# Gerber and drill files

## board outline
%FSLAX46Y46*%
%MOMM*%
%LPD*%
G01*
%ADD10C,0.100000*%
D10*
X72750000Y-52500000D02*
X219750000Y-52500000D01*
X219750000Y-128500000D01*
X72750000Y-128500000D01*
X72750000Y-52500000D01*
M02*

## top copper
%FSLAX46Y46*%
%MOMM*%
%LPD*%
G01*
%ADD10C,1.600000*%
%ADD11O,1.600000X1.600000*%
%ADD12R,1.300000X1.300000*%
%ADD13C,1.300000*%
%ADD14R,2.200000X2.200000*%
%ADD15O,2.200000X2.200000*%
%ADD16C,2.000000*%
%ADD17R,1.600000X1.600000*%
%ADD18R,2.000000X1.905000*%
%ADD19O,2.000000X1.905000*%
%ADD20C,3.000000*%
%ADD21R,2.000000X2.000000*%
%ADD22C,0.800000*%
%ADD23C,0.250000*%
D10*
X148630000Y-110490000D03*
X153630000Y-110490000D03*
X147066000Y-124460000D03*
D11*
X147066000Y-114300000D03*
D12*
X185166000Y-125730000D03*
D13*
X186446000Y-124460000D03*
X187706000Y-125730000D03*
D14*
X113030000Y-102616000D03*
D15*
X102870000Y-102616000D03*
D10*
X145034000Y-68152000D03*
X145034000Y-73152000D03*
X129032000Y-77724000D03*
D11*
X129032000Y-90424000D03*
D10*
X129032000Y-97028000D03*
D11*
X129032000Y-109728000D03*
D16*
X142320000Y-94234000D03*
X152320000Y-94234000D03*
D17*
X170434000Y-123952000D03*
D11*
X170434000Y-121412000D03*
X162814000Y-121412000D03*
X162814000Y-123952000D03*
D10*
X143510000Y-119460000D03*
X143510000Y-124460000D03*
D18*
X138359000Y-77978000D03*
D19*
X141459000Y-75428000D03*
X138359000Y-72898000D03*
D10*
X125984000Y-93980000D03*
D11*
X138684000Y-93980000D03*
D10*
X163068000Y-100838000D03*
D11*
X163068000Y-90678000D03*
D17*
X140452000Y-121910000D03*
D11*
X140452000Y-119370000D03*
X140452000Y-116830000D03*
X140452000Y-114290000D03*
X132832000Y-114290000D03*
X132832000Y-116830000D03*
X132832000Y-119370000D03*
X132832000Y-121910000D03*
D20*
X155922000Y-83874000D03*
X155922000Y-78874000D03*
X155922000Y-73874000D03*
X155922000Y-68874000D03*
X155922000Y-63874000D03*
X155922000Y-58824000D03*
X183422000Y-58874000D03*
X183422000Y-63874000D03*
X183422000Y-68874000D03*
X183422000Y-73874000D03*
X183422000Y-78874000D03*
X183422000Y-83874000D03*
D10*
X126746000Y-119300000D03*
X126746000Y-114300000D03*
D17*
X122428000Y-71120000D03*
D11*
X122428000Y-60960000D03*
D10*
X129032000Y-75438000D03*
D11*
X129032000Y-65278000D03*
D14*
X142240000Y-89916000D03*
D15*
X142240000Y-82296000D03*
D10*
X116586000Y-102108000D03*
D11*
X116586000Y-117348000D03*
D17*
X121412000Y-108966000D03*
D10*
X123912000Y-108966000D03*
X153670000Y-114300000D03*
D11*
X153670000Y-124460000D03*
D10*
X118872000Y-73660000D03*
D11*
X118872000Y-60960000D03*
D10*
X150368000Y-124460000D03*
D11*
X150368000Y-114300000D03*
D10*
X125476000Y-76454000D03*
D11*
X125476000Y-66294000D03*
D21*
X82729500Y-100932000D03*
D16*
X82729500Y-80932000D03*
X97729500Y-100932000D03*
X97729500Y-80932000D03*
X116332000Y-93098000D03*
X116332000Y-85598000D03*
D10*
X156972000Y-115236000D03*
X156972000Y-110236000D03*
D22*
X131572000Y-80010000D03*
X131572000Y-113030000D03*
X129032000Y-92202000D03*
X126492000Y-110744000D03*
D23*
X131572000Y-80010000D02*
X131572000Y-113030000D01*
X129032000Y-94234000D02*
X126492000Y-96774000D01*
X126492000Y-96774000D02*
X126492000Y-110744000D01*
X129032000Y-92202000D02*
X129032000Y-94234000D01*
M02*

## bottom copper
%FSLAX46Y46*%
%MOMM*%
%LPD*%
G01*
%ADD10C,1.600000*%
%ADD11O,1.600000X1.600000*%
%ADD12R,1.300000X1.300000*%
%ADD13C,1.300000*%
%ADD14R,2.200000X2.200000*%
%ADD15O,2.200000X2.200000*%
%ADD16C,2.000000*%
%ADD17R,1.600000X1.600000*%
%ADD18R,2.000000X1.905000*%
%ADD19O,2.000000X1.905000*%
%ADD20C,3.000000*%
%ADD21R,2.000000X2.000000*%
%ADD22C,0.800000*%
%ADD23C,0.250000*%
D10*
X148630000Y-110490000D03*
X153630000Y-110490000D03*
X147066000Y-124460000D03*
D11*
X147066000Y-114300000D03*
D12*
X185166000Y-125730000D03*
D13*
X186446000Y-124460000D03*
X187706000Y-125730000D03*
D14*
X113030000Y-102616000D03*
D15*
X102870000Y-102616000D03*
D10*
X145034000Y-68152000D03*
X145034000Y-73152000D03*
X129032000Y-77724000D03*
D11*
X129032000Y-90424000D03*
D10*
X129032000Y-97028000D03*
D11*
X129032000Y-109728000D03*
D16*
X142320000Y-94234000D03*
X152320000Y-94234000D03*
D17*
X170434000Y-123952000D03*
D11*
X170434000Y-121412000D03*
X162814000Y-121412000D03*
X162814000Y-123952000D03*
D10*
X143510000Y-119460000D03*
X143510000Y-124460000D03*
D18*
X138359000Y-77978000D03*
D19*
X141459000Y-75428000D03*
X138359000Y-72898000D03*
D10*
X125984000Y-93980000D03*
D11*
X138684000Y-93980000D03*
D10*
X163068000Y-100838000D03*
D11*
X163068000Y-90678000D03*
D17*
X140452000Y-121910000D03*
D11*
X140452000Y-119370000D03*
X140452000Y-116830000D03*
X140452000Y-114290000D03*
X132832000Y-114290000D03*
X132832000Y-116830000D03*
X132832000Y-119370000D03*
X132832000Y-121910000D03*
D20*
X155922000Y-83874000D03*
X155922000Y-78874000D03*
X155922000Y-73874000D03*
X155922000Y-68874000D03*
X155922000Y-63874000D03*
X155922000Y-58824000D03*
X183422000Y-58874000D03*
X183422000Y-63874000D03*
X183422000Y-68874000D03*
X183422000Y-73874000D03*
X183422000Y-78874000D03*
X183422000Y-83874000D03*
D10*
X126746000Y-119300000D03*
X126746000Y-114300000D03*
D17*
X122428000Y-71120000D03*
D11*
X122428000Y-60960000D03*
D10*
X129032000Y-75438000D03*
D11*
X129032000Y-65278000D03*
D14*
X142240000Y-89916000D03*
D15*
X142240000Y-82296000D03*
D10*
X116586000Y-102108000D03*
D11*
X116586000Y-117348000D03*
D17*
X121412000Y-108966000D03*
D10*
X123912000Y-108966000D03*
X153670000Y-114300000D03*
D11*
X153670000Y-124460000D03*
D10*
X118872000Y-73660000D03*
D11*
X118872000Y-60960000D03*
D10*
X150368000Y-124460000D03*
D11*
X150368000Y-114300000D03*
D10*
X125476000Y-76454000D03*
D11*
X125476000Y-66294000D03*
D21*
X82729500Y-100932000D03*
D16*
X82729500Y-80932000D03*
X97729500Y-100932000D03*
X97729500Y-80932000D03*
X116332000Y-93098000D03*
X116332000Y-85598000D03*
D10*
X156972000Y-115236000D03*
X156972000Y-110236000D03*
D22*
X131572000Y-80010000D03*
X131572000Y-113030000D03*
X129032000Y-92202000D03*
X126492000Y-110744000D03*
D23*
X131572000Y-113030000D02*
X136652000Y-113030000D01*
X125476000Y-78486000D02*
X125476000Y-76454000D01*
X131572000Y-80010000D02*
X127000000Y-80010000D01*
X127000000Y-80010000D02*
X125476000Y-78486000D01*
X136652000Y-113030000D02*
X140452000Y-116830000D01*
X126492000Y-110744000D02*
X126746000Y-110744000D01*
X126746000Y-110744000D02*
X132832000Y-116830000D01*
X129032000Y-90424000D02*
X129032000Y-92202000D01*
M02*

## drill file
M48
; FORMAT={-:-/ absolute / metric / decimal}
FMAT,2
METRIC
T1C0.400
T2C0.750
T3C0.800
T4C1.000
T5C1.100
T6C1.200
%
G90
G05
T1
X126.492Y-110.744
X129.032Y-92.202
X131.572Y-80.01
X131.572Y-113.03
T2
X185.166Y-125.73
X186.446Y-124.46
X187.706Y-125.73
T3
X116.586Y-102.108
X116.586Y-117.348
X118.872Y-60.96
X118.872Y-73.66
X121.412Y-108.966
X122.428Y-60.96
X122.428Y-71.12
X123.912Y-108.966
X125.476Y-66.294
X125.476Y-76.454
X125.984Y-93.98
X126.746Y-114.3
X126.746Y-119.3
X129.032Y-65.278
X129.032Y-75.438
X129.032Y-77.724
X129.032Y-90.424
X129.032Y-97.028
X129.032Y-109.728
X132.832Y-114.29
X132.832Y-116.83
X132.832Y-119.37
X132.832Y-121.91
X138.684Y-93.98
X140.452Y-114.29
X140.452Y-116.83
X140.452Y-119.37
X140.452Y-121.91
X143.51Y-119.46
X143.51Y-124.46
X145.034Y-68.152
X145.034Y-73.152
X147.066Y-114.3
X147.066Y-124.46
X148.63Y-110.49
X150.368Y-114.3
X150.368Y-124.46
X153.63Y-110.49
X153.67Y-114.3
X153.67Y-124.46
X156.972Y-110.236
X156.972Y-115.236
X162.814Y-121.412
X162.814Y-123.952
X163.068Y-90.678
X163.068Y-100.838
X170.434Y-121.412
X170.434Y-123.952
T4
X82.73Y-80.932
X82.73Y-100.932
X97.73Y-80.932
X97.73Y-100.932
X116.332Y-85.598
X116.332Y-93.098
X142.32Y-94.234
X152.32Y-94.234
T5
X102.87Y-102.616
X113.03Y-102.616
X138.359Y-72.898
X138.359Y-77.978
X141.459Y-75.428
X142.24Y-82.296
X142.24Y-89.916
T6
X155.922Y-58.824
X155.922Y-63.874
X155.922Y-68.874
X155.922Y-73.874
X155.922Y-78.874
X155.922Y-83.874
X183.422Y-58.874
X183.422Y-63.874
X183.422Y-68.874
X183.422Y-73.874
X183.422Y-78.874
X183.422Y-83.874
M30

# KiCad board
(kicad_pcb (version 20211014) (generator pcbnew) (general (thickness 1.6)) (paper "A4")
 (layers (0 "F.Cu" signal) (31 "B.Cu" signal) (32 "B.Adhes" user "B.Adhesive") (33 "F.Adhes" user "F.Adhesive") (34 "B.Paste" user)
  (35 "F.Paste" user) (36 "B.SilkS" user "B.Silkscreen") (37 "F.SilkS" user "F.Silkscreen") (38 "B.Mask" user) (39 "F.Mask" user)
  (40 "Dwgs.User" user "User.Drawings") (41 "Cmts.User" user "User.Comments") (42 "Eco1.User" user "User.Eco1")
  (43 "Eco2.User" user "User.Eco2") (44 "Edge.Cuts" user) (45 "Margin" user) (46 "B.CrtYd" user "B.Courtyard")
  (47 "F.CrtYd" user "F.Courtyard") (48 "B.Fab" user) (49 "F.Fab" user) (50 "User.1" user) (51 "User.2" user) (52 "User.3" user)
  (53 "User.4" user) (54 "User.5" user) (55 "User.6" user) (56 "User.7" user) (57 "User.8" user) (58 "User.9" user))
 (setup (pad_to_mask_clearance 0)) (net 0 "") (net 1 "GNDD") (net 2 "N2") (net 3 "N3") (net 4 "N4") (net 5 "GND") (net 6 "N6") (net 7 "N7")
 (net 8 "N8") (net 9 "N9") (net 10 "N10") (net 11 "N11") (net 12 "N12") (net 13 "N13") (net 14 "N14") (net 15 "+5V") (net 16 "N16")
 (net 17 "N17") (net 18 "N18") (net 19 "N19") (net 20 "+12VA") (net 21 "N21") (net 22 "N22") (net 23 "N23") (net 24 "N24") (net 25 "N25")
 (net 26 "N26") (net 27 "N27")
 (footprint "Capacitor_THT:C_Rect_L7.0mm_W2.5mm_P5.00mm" (layer "F.Cu") (at 148.63 110.49)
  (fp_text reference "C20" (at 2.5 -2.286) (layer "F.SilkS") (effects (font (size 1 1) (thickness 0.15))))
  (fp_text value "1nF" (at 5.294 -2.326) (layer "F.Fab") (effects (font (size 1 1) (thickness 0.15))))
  (pad "1" thru_hole circle (at 0 0) (size 1.6 1.6) (drill 0.8) (layers *.Cu *.Mask) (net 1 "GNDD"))
  (pad "2" thru_hole circle (at 5 0) (size 1.6 1.6) (drill 0.8) (layers *.Cu *.Mask) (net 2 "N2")))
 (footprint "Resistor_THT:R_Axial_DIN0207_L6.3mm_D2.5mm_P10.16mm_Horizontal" (layer "F.Cu") (at 147.066 124.46 90)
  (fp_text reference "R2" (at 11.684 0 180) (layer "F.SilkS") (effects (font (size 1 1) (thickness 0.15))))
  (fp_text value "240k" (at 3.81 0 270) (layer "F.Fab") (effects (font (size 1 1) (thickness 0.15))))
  (pad "1" thru_hole circle (at 0 0 90) (size 1.6 1.6) (drill 0.8) (layers *.Cu *.Mask) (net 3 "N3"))
  (pad "2" thru_hole oval (at 10.16 0 90) (size 1.6 1.6) (drill 0.8) (layers *.Cu *.Mask) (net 2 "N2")))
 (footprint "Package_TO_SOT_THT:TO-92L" (layer "F.Cu") (at 185.166 125.73)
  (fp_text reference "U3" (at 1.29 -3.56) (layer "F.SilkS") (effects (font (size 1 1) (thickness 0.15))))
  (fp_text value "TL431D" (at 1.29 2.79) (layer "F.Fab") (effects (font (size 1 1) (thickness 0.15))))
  (pad "1" thru_hole rect (at 0 0) (size 1.3 1.3) (drill 0.75) (layers *.Cu *.Mask) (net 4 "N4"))
  (pad "2" thru_hole circle (at 1.28 -1.27) (size 1.3 1.3) (drill 0.75) (layers *.Cu *.Mask) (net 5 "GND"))
  (pad "3" thru_hole circle (at 2.54 0) (size 1.3 1.3) (drill 0.75) (layers *.Cu *.Mask) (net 5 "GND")))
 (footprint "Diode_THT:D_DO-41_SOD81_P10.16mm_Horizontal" (layer "F.Cu") (at 113.03 102.616 180)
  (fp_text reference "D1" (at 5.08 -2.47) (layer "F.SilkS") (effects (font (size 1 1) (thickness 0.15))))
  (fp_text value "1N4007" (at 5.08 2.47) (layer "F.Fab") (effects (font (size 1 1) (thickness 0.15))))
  (pad "1" thru_hole rect (at 0 0 180) (size 2.2 2.2) (drill 1.1) (layers *.Cu *.Mask) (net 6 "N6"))
  (pad "2" thru_hole oval (at 10.16 0 180) (size 2.2 2.2) (drill 1.1) (layers *.Cu *.Mask) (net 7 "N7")))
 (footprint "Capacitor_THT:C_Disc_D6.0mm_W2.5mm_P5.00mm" (layer "F.Cu") (at 145.034 68.152 -90)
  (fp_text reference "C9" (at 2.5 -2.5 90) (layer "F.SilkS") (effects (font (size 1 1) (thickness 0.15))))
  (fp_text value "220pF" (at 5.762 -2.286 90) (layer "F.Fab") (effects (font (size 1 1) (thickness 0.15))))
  (pad "1" thru_hole circle (at 0 0 270) (size 1.6 1.6) (drill 0.8) (layers *.Cu *.Mask) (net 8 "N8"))
  (pad "2" thru_hole circle (at 5 0 270) (size 1.6 1.6) (drill 0.8) (layers *.Cu *.Mask) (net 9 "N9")))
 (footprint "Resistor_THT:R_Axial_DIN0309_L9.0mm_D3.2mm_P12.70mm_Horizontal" (layer "F.Cu") (at 129.032 77.724 -90)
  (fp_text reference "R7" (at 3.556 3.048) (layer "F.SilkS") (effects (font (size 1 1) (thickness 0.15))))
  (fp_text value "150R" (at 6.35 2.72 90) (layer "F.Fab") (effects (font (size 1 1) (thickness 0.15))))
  (pad "1" thru_hole circle (at 0 0 270) (size 1.6 1.6) (drill 0.8) (layers *.Cu *.Mask) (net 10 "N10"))
  (pad "2" thru_hole oval (at 12.7 0 270) (size 1.6 1.6) (drill 0.8) (layers *.Cu *.Mask) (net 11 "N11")))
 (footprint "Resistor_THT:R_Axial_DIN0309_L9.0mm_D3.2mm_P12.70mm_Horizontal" (layer "F.Cu") (at 129.032 97.028 -90)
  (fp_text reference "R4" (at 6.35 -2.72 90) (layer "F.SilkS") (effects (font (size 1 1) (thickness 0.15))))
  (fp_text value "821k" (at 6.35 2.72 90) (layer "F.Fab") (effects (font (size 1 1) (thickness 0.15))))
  (pad "1" thru_hole circle (at 0 0 270) (size 1.6 1.6) (drill 0.8) (layers *.Cu *.Mask) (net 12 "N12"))
  (pad "2" thru_hole oval (at 12.7 0 270) (size 1.6 1.6) (drill 0.8) (layers *.Cu *.Mask) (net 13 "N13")))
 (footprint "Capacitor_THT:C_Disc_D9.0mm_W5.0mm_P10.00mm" (layer "F.Cu") (at 142.32 94.234)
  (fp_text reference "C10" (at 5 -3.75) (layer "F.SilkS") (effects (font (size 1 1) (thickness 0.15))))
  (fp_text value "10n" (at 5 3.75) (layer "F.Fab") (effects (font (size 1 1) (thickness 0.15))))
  (pad "1" thru_hole circle (at 0 0) (size 2 2) (drill 1) (layers *.Cu *.Mask) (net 12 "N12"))
  (pad "2" thru_hole circle (at 10 0) (size 2 2) (drill 1) (layers *.Cu *.Mask) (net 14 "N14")))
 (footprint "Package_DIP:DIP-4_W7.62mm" (layer "F.Cu") (at 170.434 123.952 180)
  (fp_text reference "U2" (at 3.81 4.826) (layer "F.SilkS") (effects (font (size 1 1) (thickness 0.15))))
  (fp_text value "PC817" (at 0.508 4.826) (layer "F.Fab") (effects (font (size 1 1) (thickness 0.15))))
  (pad "1" thru_hole rect (at 0 0 180) (size 1.6 1.6) (drill 0.8) (layers *.Cu *.Mask) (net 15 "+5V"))
  (pad "2" thru_hole oval (at 0 2.54 180) (size 1.6 1.6) (drill 0.8) (layers *.Cu *.Mask) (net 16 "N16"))
  (pad "3" thru_hole oval (at 7.62 2.54 180) (size 1.6 1.6) (drill 0.8) (layers *.Cu *.Mask) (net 1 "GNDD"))
  (pad "4" thru_hole oval (at 7.62 0 180) (size 1.6 1.6) (drill 0.8) (layers *.Cu *.Mask) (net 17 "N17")))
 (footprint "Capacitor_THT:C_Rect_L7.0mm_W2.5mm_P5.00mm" (layer "F.Cu") (at 143.51 119.46 -90)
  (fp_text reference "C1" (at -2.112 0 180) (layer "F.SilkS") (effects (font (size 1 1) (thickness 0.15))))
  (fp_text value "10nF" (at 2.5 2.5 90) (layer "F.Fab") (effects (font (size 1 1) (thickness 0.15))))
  (pad "1" thru_hole circle (at 0 0 270) (size 1.6 1.6) (drill 0.8) (layers *.Cu *.Mask) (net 1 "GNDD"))
  (pad "2" thru_hole circle (at 5 0 270) (size 1.6 1.6) (drill 0.8) (layers *.Cu *.Mask) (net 17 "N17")))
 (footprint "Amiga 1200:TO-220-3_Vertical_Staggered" (layer "F.Cu") (at 138.359 77.978 90)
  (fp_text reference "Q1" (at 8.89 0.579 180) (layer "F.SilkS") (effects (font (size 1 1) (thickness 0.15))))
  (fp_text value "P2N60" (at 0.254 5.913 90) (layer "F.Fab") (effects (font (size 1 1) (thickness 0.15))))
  (pad "1" thru_hole rect (at 0 0 90) (size 1.905 2) (drill 1.1) (layers *.Cu *.Mask) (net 10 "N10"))
  (pad "2" thru_hole oval (at 2.55 3.1 90) (size 1.905 2) (drill 1.1) (layers *.Cu *.Mask) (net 9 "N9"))
  (pad "3" thru_hole oval (at 5.08 0 90) (size 1.905 2) (drill 1.1) (layers *.Cu *.Mask) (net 8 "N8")))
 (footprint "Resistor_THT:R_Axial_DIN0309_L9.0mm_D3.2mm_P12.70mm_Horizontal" (layer "F.Cu") (at 125.984 93.98)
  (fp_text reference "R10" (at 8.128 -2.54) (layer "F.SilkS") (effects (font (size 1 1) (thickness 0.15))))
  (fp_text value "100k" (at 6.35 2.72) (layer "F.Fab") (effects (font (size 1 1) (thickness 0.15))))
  (pad "1" thru_hole circle (at 0 0) (size 1.6 1.6) (drill 0.8) (layers *.Cu *.Mask) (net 12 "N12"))
  (pad "2" thru_hole oval (at 12.7 0) (size 1.6 1.6) (drill 0.8) (layers *.Cu *.Mask) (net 14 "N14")))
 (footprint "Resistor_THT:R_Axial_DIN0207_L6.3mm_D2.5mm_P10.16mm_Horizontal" (layer "F.Cu") (at 163.068 100.838 90)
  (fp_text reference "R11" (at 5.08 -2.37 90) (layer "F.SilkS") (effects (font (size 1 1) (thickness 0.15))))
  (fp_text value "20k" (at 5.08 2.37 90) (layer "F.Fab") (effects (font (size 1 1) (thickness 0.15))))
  (pad "1" thru_hole circle (at 0 0 90) (size 1.6 1.6) (drill 0.8) (layers *.Cu *.Mask) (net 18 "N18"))
  (pad "2" thru_hole oval (at 10.16 0 90) (size 1.6 1.6) (drill 0.8) (layers *.Cu *.Mask) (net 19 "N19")))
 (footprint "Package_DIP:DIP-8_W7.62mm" (layer "F.Cu") (at 140.452 121.91 180)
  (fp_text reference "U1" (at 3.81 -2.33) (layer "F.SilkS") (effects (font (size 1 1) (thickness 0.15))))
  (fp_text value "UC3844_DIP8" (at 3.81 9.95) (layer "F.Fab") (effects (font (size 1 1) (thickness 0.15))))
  (pad "1" thru_hole rect (at 0 0 180) (size 1.6 1.6) (drill 0.8) (layers *.Cu *.Mask) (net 17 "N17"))
  (pad "2" thru_hole oval (at 0 2.54 180) (size 1.6 1.6) (drill 0.8) (layers *.Cu *.Mask) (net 1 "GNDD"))
  (pad "3" thru_hole oval (at 0 5.08 180) (size 1.6 1.6) (drill 0.8) (layers *.Cu *.Mask) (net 13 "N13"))
  (pad "4" thru_hole oval (at 0 7.62 180) (size 1.6 1.6) (drill 0.8) (layers *.Cu *.Mask) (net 2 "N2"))
  (pad "5" thru_hole oval (at 7.62 7.62 180) (size 1.6 1.6) (drill 0.8) (layers *.Cu *.Mask) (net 1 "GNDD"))
  (pad "6" thru_hole oval (at 7.62 5.08 180) (size 1.6 1.6) (drill 0.8) (layers *.Cu *.Mask) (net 11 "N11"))
  (pad "7" thru_hole oval (at 7.62 2.54 180) (size 1.6 1.6) (drill 0.8) (layers *.Cu *.Mask) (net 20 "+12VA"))
  (pad "8" thru_hole oval (at 7.62 0 180) (size 1.6 1.6) (drill 0.8) (layers *.Cu *.Mask) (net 3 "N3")))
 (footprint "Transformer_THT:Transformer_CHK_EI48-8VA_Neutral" (layer "F.Cu") (at 155.922 83.874)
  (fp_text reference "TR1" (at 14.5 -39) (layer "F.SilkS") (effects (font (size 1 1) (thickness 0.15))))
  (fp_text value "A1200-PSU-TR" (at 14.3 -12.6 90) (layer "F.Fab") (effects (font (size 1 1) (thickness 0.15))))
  (pad "1" thru_hole circle (at 0 0) (size 3 3) (drill 1.2) (layers *.Cu *.Mask) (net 12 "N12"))
  (pad "2" thru_hole circle (at 0 -5) (size 3 3) (drill 1.2) (layers *.Cu *.Mask))
  (pad "3" thru_hole circle (at 0 -10) (size 3 3) (drill 1.2) (layers *.Cu *.Mask) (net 9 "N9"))
  (pad "4" thru_hole circle (at 0 -15) (size 3 3) (drill 1.2) (layers *.Cu *.Mask))
  (pad "5" thru_hole circle (at 0 -20) (size 3 3) (drill 1.2) (layers *.Cu *.Mask) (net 19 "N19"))
  (pad "6" thru_hole circle (at 0 -25.05) (size 3 3) (drill 1.2) (layers *.Cu *.Mask) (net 1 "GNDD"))
  (pad "7" thru_hole circle (at 27.5 -25) (size 3 3) (drill 1.2) (layers *.Cu *.Mask) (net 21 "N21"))
  (pad "8" thru_hole circle (at 27.5 -20) (size 3 3) (drill 1.2) (layers *.Cu *.Mask) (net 5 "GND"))
  (pad "9" thru_hole circle (at 27.5 -15) (size 3 3) (drill 1.2) (layers *.Cu *.Mask) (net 5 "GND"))
  (pad "10" thru_hole circle (at 27.5 -10) (size 3 3) (drill 1.2) (layers *.Cu *.Mask) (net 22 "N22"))
  (pad "11" thru_hole circle (at 27.5 -5) (size 3 3) (drill 1.2) (layers *.Cu *.Mask) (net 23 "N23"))
  (pad "12" thru_hole circle (at 27.5 0) (size 3 3) (drill 1.2) (layers *.Cu *.Mask) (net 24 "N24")))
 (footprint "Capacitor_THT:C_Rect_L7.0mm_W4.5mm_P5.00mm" (layer "F.Cu") (at 126.746 119.3 90)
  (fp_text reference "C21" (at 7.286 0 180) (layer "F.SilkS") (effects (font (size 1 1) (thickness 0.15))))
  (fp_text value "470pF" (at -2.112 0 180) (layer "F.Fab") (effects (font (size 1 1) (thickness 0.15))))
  (pad "1" thru_hole circle (at 0 0 90) (size 1.6 1.6) (drill 0.8) (layers *.Cu *.Mask) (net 13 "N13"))
  (pad "2" thru_hole circle (at 5 0 90) (size 1.6 1.6) (drill 0.8) (layers *.Cu *.Mask) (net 1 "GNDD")))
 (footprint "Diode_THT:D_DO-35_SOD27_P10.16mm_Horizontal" (layer "F.Cu") (at 122.428 71.12 90)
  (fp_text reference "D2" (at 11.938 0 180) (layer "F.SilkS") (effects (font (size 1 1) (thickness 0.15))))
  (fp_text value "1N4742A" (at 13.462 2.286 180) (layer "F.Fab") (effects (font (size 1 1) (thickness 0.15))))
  (pad "1" thru_hole rect (at 0 0 90) (size 1.6 1.6) (drill 0.8) (layers *.Cu *.Mask) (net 8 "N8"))
  (pad "2" thru_hole oval (at 10.16 0 90) (size 1.6 1.6) (drill 0.8) (layers *.Cu *.Mask) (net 1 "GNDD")))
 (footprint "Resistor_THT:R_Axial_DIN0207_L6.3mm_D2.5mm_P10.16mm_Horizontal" (layer "F.Cu") (at 129.032 75.438 90)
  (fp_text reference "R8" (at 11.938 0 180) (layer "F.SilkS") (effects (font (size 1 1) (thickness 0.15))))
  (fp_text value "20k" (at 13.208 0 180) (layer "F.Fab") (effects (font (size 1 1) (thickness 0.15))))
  (pad "1" thru_hole circle (at 0 0 90) (size 1.6 1.6) (drill 0.8) (layers *.Cu *.Mask) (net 10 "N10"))
  (pad "2" thru_hole oval (at 10.16 0 90) (size 1.6 1.6) (drill 0.8) (layers *.Cu *.Mask) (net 1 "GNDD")))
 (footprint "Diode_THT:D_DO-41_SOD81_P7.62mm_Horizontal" (layer "F.Cu") (at 142.24 89.916 90)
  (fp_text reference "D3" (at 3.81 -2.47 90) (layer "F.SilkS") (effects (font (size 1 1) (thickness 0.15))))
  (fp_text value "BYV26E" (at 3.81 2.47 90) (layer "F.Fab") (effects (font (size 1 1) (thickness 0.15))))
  (pad "1" thru_hole rect (at 0 0 90) (size 2.2 2.2) (drill 1.1) (layers *.Cu *.Mask) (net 14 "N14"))
  (pad "2" thru_hole oval (at 7.62 0 90) (size 2.2 2.2) (drill 1.1) (layers *.Cu *.Mask) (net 9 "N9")))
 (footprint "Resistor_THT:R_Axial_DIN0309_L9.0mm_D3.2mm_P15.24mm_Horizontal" (layer "F.Cu") (at 116.586 102.108 -90)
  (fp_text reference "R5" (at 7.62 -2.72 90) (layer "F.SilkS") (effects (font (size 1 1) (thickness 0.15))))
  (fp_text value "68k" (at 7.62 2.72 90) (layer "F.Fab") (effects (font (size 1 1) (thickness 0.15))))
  (pad "1" thru_hole circle (at 0 0 270) (size 1.6 1.6) (drill 0.8) (layers *.Cu *.Mask) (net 6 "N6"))
  (pad "2" thru_hole oval (at 15.24 0 270) (size 1.6 1.6) (drill 0.8) (layers *.Cu *.Mask) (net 20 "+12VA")))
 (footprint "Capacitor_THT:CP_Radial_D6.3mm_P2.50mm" (layer "F.Cu") (at 121.412 108.966)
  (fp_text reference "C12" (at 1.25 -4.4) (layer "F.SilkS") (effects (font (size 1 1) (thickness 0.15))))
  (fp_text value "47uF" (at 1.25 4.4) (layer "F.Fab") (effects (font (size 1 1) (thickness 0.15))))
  (pad "1" thru_hole rect (at 0 0) (size 1.6 1.6) (drill 0.8) (layers *.Cu *.Mask) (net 20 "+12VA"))
  (pad "2" thru_hole circle (at 2.5 0) (size 1.6 1.6) (drill 0.8) (layers *.Cu *.Mask) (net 1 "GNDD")))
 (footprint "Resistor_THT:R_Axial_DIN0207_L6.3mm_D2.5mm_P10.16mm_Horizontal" (layer "F.Cu") (at 153.67 114.3 -90)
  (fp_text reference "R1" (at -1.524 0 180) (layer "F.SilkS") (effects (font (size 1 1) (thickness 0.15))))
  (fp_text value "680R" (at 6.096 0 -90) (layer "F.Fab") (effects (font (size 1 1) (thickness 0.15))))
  (pad "1" thru_hole circle (at 0 0 270) (size 1.6 1.6) (drill 0.8) (layers *.Cu *.Mask) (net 3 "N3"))
  (pad "2" thru_hole oval (at 10.16 0 270) (size 1.6 1.6) (drill 0.8) (layers *.Cu *.Mask) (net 17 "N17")))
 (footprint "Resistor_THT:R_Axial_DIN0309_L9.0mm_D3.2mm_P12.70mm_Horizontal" (layer "F.Cu") (at 118.872 73.66 90)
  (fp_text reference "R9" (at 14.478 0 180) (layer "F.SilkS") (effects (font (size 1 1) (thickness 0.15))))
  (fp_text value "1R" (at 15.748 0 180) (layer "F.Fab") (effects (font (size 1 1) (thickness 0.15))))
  (pad "1" thru_hole circle (at 0 0 90) (size 1.6 1.6) (drill 0.8) (layers *.Cu *.Mask) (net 8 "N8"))
  (pad "2" thru_hole oval (at 12.7 0 90) (size 1.6 1.6) (drill 0.8) (layers *.Cu *.Mask) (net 1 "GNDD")))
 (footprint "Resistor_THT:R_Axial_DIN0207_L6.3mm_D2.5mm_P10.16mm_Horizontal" (layer "F.Cu") (at 150.368 124.46 90)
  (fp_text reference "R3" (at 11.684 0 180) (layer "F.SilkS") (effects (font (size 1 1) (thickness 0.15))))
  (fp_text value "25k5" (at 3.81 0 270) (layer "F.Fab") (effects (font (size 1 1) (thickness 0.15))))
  (pad "1" thru_hole circle (at 0 0 90) (size 1.6 1.6) (drill 0.8) (layers *.Cu *.Mask) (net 3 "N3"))
  (pad "2" thru_hole oval (at 10.16 0 90) (size 1.6 1.6) (drill 0.8) (layers *.Cu *.Mask) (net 2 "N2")))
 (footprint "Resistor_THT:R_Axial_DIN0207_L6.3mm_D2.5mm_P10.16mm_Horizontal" (layer "F.Cu") (at 125.476 76.454 90)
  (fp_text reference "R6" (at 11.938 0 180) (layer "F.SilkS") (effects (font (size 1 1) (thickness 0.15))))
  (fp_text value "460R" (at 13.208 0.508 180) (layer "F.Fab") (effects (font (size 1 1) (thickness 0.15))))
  (pad "1" thru_hole circle (at 0 0 90) (size 1.6 1.6) (drill 0.8) (layers *.Cu *.Mask) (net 13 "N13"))
  (pad "2" thru_hole oval (at 10.16 0 90) (size 1.6 1.6) (drill 0.8) (layers *.Cu *.Mask) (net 8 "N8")))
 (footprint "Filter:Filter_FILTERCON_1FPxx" (layer "F.Cu") (at 82.7295 100.932 90)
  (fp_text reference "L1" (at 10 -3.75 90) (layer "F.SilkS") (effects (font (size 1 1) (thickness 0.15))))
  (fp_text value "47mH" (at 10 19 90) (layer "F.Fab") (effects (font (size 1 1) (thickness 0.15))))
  (pad "1" thru_hole rect (at 0 0 90) (size 2 2) (drill 1) (layers *.Cu *.Mask) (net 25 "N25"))
  (pad "2" thru_hole circle (at 20 0 90) (size 2 2) (drill 1) (layers *.Cu *.Mask) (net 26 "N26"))
  (pad "3" thru_hole circle (at 0 15 90) (size 2 2) (drill 1) (layers *.Cu *.Mask) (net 7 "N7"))
  (pad "4" thru_hole circle (at 20 15 90) (size 2 2) (drill 1) (layers *.Cu *.Mask) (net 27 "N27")))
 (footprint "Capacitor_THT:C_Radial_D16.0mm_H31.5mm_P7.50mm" (layer "F.Cu") (at 116.332 93.098 90)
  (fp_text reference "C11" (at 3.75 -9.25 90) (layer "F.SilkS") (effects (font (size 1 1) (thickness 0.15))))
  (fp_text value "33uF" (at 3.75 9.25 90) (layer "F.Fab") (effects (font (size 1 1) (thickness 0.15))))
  (pad "1" thru_hole circle (at 0 0 90) (size 2 2) (drill 1) (layers *.Cu *.Mask) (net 12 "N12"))
  (pad "2" thru_hole circle (at 7.5 0 90) (size 2 2) (drill 1) (layers *.Cu *.Mask) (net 1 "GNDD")))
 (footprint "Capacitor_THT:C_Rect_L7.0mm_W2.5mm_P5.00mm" (layer "F.Cu") (at 156.972 115.236 90)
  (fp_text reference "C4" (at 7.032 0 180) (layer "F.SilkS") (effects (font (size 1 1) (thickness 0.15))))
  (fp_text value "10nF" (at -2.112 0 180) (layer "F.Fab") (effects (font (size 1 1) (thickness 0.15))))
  (pad "1" thru_hole circle (at 0 0 90) (size 1.6 1.6) (drill 0.8) (layers *.Cu *.Mask) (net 17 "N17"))
  (pad "2" thru_hole circle (at 5 0 90) (size 1.6 1.6) (drill 0.8) (layers *.Cu *.Mask) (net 2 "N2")))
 (gr_rect (start 72.75 52.5) (end 219.75 128.5) (layer "Edge.Cuts") (width 0.1) (fill none))
 (segment (start 131.572 80.01) (end 131.572 113.03) (width 0.25) (layer "F.Cu") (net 13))
 (via (at 131.572 80.01) (size 0.8) (drill 0.4) (layers "F.Cu" "B.Cu") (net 13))
 (via (at 131.572 113.03) (size 0.8) (drill 0.4) (layers "F.Cu" "B.Cu") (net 13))
 (segment (start 131.572 113.03) (end 136.652 113.03) (width 0.25) (layer "B.Cu") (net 13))
 (segment (start 125.476 78.486) (end 125.476 76.454) (width 0.25) (layer "B.Cu") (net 13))
 (segment (start 131.572 80.01) (end 127 80.01) (width 0.25) (layer "B.Cu") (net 13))
 (segment (start 127 80.01) (end 125.476 78.486) (width 0.25) (layer "B.Cu") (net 13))
 (segment (start 136.652 113.03) (end 140.452 116.83) (width 0.25) (layer "B.Cu") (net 13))
 (segment (start 129.032 94.234) (end 126.492 96.774) (width 0.25) (layer "F.Cu") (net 11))
 (segment (start 126.492 96.774) (end 126.492 110.744) (width 0.25) (layer "F.Cu") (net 11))
 (segment (start 129.032 92.202) (end 129.032 94.234) (width 0.25) (layer "F.Cu") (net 11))
 (via (at 129.032 92.202) (size 0.8) (drill 0.4) (layers "F.Cu" "B.Cu") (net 11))
 (via (at 126.492 110.744) (size 0.8) (drill 0.4) (layers "F.Cu" "B.Cu") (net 11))
 (segment (start 126.492 110.744) (end 126.746 110.744) (width 0.25) (layer "B.Cu") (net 11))
 (segment (start 126.746 110.744) (end 132.832 116.83) (width 0.25) (layer "B.Cu") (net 11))
 (segment (start 129.032 90.424) (end 129.032 92.202) (width 0.25) (layer "B.Cu") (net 11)))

